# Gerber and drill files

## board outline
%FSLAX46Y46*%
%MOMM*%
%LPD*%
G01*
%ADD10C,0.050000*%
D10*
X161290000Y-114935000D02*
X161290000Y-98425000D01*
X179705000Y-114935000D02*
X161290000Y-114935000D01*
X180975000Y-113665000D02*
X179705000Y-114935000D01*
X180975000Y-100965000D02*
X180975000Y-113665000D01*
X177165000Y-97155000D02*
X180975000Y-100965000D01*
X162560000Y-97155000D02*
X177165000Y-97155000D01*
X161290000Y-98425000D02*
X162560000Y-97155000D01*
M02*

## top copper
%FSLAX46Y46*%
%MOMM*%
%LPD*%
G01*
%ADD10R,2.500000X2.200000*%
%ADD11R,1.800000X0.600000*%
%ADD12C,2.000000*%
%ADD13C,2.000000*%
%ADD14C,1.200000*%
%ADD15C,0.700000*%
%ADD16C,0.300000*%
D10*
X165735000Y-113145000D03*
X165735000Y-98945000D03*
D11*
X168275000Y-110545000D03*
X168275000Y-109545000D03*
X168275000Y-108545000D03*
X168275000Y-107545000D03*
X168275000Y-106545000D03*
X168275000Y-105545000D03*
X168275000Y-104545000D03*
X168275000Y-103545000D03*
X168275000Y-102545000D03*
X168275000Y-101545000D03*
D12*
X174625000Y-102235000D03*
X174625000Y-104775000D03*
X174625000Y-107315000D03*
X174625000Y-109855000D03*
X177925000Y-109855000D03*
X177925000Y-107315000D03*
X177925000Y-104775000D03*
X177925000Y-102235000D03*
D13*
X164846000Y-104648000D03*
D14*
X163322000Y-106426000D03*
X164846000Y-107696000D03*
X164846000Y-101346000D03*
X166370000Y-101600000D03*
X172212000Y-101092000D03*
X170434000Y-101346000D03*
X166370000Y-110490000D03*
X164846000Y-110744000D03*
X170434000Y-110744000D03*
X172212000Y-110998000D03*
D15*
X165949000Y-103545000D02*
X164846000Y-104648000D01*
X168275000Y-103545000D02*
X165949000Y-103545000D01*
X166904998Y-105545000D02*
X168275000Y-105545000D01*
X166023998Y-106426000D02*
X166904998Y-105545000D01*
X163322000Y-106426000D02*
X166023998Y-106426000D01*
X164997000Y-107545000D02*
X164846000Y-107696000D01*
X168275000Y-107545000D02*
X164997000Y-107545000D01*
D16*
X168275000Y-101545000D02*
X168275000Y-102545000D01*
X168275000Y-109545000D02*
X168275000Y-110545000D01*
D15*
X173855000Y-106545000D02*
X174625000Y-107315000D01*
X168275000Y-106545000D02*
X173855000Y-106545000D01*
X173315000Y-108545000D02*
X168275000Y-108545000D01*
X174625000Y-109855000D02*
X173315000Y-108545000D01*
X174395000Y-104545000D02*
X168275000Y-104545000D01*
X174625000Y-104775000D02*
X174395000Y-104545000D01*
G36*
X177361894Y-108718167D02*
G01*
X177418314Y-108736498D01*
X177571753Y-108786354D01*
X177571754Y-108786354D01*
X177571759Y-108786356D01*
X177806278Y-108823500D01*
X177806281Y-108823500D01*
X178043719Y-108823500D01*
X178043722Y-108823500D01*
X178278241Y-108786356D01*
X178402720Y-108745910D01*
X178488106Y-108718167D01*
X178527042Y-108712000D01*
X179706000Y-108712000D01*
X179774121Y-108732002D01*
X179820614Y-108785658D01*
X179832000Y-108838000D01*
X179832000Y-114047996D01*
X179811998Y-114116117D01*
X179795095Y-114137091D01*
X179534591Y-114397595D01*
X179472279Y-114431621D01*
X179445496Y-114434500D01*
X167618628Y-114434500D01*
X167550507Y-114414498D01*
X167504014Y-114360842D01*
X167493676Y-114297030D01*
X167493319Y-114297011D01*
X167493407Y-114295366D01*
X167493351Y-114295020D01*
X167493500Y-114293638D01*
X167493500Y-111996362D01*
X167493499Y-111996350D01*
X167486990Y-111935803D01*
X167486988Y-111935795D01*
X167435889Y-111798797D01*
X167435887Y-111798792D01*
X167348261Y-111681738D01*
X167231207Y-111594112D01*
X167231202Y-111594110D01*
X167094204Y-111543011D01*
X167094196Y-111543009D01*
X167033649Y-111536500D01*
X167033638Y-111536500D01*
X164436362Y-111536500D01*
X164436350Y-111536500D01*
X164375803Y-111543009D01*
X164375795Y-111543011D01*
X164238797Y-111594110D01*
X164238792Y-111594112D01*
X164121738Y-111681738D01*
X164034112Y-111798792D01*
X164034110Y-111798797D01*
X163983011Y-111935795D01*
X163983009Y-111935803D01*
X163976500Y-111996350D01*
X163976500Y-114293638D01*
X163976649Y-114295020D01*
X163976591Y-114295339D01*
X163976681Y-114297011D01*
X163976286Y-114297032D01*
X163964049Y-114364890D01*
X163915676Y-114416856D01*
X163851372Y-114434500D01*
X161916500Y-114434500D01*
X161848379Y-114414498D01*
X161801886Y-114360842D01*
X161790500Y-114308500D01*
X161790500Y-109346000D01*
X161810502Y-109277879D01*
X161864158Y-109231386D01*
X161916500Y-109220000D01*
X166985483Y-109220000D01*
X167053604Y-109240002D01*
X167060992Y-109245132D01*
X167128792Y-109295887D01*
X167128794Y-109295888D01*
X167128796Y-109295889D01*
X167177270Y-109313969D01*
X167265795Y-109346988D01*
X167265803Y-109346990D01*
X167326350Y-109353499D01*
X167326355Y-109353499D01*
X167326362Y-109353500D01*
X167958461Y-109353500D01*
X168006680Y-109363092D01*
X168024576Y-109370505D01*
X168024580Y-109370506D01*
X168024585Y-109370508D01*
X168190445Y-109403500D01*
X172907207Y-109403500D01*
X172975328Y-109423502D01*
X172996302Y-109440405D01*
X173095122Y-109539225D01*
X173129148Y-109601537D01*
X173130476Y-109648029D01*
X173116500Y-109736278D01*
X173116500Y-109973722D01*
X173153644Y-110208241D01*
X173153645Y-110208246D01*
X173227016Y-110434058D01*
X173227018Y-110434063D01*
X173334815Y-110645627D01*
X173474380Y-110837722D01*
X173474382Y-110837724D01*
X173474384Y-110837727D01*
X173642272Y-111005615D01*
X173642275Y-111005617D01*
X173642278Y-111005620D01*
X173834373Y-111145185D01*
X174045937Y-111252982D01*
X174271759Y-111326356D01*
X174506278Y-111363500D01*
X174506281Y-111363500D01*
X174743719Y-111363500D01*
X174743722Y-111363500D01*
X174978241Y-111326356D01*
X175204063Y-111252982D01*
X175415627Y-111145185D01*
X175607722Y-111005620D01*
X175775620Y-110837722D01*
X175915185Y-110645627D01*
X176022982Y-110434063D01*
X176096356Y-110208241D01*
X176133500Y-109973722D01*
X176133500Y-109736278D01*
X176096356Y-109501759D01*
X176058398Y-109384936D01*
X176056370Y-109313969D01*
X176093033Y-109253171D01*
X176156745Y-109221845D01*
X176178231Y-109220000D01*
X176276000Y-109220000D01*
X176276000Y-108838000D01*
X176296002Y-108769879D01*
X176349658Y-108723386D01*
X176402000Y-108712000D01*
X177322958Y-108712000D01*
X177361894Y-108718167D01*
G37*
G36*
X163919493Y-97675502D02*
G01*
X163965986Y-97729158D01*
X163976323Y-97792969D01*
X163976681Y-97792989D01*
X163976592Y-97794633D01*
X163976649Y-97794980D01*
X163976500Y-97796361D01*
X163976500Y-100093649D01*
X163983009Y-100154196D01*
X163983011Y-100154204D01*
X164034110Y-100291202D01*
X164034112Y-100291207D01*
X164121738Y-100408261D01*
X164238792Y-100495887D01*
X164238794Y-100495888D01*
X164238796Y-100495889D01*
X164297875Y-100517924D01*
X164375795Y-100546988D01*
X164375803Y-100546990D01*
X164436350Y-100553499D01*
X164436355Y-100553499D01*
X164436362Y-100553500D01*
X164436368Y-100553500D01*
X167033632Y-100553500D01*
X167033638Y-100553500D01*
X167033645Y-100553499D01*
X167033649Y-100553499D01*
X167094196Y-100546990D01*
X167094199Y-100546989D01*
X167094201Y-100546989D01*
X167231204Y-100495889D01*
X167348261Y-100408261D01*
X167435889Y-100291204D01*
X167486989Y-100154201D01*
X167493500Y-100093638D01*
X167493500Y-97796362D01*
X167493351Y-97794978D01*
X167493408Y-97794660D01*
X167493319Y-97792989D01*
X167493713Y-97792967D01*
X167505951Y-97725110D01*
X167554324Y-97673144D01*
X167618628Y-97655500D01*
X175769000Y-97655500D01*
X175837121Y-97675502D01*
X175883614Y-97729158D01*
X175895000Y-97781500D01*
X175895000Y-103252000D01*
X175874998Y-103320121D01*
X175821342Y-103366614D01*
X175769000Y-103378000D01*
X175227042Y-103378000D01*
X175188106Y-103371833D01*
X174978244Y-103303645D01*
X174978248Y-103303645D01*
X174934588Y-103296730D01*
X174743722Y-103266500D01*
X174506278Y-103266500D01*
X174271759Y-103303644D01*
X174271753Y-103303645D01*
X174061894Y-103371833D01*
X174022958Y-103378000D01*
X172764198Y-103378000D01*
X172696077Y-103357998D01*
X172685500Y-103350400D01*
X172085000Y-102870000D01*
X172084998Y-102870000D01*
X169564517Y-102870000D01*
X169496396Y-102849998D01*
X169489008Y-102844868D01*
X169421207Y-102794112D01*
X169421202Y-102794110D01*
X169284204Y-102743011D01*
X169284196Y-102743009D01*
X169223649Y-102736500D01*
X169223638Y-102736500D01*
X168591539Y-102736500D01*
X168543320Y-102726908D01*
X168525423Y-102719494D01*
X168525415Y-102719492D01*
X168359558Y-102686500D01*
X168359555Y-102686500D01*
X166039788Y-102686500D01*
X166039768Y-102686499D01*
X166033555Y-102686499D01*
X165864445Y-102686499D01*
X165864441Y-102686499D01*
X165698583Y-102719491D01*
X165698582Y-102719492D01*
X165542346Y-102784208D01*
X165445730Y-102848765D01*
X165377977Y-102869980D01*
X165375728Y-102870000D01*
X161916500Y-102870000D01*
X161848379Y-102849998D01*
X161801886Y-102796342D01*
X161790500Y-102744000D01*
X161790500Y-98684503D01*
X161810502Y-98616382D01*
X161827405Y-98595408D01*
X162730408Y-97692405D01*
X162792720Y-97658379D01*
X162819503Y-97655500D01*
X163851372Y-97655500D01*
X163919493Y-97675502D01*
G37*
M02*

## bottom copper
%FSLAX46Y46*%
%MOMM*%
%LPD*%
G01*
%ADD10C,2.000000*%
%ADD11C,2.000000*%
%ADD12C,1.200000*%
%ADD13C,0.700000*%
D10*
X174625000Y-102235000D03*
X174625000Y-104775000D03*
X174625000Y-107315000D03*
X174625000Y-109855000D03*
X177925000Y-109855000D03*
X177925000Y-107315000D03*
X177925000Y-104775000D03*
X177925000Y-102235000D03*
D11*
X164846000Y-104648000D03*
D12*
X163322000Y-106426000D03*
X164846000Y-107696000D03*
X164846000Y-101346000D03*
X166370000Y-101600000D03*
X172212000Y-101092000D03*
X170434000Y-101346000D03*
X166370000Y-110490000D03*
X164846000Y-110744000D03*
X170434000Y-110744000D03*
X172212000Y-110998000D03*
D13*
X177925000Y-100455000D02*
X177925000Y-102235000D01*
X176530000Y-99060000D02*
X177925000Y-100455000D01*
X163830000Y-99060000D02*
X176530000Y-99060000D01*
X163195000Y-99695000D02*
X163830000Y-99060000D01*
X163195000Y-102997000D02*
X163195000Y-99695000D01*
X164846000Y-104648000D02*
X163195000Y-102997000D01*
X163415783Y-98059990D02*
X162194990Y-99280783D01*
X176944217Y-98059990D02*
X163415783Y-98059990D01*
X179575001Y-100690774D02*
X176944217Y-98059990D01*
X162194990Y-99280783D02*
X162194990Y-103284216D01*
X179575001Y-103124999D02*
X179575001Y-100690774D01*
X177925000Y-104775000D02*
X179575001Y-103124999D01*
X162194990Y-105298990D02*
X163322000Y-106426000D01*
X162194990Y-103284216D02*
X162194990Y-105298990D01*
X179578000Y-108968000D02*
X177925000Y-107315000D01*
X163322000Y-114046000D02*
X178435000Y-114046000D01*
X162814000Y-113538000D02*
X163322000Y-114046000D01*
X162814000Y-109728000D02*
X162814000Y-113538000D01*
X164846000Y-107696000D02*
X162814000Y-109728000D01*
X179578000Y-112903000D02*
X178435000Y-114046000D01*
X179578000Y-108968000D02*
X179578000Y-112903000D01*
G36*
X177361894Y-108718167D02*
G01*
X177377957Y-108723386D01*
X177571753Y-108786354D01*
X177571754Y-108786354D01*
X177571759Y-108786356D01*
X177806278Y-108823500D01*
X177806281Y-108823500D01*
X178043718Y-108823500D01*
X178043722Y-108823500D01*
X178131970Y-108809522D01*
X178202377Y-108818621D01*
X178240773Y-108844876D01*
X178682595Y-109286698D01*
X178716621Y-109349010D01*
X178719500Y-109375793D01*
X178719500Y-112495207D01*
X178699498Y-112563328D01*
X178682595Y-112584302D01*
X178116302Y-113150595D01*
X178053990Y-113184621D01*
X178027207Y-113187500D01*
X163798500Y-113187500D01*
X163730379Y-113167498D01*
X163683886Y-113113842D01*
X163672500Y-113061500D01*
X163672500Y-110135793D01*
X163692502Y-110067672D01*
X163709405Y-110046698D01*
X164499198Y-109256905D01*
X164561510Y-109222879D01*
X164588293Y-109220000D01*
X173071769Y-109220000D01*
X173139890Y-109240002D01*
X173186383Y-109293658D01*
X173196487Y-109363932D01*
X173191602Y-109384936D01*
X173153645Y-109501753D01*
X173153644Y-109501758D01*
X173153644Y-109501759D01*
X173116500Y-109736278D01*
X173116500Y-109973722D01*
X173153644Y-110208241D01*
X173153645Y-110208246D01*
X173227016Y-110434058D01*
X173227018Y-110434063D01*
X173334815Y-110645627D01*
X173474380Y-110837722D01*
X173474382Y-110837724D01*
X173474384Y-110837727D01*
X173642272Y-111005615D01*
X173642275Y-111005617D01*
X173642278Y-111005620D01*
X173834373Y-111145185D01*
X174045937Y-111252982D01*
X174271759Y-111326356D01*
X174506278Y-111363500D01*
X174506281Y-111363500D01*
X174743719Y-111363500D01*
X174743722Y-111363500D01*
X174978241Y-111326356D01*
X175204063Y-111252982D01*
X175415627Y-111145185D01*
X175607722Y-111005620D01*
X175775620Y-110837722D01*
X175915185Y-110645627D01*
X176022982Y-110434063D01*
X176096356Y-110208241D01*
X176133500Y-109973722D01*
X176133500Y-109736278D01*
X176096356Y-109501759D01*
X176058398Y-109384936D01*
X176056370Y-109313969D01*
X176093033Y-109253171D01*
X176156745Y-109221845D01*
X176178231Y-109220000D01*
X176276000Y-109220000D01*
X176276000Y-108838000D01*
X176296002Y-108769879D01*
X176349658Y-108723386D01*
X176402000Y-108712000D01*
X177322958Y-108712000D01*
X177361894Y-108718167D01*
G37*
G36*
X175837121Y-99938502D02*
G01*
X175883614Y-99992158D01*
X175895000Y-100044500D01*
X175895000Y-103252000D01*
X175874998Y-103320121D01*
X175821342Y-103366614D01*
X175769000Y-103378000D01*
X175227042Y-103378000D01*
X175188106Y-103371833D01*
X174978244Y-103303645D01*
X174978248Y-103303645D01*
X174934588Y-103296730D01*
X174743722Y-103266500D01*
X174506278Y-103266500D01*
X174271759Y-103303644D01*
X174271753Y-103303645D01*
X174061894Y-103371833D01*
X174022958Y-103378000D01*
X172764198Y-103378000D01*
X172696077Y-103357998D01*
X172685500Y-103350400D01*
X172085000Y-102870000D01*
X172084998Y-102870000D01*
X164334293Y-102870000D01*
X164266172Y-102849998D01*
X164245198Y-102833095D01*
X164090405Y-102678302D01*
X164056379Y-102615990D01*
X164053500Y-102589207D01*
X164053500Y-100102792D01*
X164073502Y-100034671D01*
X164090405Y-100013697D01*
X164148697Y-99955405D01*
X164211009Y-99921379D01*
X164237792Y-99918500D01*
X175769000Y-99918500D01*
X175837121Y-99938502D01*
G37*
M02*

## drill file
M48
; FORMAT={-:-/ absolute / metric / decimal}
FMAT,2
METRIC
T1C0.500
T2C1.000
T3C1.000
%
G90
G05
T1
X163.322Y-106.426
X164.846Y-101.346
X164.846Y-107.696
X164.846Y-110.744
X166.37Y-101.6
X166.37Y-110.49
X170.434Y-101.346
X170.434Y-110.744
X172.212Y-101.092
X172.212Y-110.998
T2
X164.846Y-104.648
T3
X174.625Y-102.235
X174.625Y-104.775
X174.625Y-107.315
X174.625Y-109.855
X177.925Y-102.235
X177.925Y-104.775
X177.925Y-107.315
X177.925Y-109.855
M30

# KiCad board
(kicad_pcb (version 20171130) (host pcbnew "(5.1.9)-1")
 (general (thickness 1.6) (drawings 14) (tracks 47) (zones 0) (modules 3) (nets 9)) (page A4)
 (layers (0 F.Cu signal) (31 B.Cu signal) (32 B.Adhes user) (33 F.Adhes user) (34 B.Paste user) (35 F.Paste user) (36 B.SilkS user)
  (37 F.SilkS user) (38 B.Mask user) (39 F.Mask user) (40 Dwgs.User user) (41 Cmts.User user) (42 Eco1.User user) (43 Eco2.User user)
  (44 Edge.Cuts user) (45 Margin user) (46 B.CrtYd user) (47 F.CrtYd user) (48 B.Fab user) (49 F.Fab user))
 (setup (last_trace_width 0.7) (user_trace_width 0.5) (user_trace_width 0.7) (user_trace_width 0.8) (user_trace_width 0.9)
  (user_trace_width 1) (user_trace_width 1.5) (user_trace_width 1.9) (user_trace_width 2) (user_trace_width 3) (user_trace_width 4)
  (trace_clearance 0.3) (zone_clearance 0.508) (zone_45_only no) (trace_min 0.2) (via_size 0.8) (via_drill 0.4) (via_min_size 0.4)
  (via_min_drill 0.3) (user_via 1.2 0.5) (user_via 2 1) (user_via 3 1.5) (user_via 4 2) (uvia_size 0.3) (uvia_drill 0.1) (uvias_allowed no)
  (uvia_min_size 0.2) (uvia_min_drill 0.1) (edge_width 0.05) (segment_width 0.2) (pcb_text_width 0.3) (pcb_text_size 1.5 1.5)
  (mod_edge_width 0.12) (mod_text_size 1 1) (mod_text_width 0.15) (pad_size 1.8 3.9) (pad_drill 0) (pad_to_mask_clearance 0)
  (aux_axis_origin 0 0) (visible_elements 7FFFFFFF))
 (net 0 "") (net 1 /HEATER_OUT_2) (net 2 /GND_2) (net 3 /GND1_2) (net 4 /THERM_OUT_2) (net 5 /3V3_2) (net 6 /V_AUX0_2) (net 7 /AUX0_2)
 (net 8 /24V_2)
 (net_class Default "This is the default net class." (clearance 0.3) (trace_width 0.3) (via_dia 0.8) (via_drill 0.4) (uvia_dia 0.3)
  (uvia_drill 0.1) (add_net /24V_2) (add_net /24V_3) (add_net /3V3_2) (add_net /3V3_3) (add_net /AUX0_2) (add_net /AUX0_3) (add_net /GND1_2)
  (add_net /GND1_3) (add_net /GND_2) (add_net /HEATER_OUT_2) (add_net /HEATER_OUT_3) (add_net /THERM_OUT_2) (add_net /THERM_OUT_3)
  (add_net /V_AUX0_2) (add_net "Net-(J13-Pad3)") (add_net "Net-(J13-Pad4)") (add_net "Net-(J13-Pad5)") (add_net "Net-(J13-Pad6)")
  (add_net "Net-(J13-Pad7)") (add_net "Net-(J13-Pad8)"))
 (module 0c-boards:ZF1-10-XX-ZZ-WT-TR (layer F.Cu) (at 168.275 106.045 270)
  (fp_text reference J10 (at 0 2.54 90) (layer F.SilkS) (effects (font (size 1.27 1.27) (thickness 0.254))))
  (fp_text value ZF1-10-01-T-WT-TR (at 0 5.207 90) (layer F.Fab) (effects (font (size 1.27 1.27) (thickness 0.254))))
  (pad 12 smd rect (at 7.1 2.54 270) (size 2.2 2.5) (layers F.Cu F.Paste F.Mask))
  (pad 11 smd rect (at -7.1 2.54 270) (size 2.2 2.5) (layers F.Cu F.Paste F.Mask))
  (pad 10 smd rect (at 4.5 0 270) (size 0.6 1.8) (layers F.Cu F.Paste F.Mask) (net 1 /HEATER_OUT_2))
  (pad 9 smd rect (at 3.5 0 270) (size 0.6 1.8) (layers F.Cu F.Paste F.Mask) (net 1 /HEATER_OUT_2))
  (pad 8 smd rect (at 2.5 0 270) (size 0.6 1.8) (layers F.Cu F.Paste F.Mask) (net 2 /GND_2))
  (pad 7 smd rect (at 1.5 0 270) (size 0.6 1.8) (layers F.Cu F.Paste F.Mask) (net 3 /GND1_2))
  (pad 6 smd rect (at 0.5 0 270) (size 0.6 1.8) (layers F.Cu F.Paste F.Mask) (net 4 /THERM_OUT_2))
  (pad 5 smd rect (at -0.5 0 270) (size 0.6 1.8) (layers F.Cu F.Paste F.Mask) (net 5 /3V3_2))
  (pad 4 smd rect (at -1.5 0 270) (size 0.6 1.8) (layers F.Cu F.Paste F.Mask) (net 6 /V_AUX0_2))
  (pad 3 smd rect (at -2.5 0 270) (size 0.6 1.8) (layers F.Cu F.Paste F.Mask) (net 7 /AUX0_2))
  (pad 2 smd rect (at -3.5 0 270) (size 0.6 1.8) (layers F.Cu F.Paste F.Mask) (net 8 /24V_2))
  (pad 1 smd rect (at -4.5 0 270) (size 0.6 1.8) (layers F.Cu F.Paste F.Mask) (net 8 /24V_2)))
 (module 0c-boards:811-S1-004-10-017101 (layer B.Cu) (at 174.625 106.045 270)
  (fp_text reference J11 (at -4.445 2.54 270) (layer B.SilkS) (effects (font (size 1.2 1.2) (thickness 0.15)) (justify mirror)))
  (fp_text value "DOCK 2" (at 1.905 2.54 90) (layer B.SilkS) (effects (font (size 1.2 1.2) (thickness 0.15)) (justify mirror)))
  (pad 1 thru_hole circle (at -3.81 0 270) (size 2 2) (drill 1) (layers *.Cu *.Mask) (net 8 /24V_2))
  (pad 2 thru_hole circle (at -1.27 0 270) (size 2 2) (drill 1) (layers *.Cu *.Mask) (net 6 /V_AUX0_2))
  (pad 3 thru_hole circle (at 1.27 0 270) (size 2 2) (drill 1) (layers *.Cu *.Mask) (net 4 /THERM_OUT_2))
  (pad 4 thru_hole circle (at 3.81 0 270) (size 2 2) (drill 1) (layers *.Cu *.Mask) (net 2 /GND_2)))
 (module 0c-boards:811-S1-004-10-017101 (layer B.Cu) (at 177.925 106.045 90)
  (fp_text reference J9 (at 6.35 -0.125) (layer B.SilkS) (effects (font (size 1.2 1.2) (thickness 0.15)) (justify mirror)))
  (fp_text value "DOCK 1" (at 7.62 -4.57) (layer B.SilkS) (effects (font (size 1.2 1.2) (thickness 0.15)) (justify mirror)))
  (pad 1 thru_hole circle (at -3.81 0 90) (size 2 2) (drill 1) (layers *.Cu *.Mask) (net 1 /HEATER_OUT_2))
  (pad 2 thru_hole circle (at -1.27 0 90) (size 2 2) (drill 1) (layers *.Cu *.Mask) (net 3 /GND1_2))
  (pad 3 thru_hole circle (at 1.27 0 90) (size 2 2) (drill 1) (layers *.Cu *.Mask) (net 5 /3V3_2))
  (pad 4 thru_hole circle (at 3.81 0 90) (size 2 2) (drill 1) (layers *.Cu *.Mask) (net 7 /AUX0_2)))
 (gr_line (start 161.29 114.935) (end 161.29 98.425) (layer Edge.Cuts) (width 0.05))
 (gr_line (start 179.705 114.935) (end 161.29 114.935) (layer Edge.Cuts) (width 0.05))
 (gr_line (start 180.975 113.665) (end 179.705 114.935) (layer Edge.Cuts) (width 0.05))
 (gr_line (start 180.975 100.965) (end 180.975 113.665) (layer Edge.Cuts) (width 0.05))
 (gr_line (start 177.165 97.155) (end 180.975 100.965) (layer Edge.Cuts) (width 0.05))
 (gr_line (start 162.56 97.155) (end 177.165 97.155) (layer Edge.Cuts) (width 0.05))
 (gr_line (start 161.29 98.425) (end 162.56 97.155) (layer Edge.Cuts) (width 0.05))
 (via (at 164.846 104.648) (size 2) (drill 1) (layers F.Cu B.Cu) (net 7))
 (segment (start 165.949 103.545) (end 164.846 104.648) (width 0.7) (layer F.Cu) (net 7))
 (segment (start 168.275 103.545) (end 165.949 103.545) (width 0.7) (layer F.Cu) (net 7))
 (segment (start 177.925 100.455) (end 177.925 102.235) (width 0.7) (layer B.Cu) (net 7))
 (segment (start 176.53 99.06) (end 177.925 100.455) (width 0.7) (layer B.Cu) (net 7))
 (segment (start 163.83 99.06) (end 176.53 99.06) (width 0.7) (layer B.Cu) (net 7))
 (segment (start 163.195 99.695) (end 163.83 99.06) (width 0.7) (layer B.Cu) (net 7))
 (segment (start 163.195 102.997) (end 163.195 99.695) (width 0.7) (layer B.Cu) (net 7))
 (segment (start 164.846 104.648) (end 163.195 102.997) (width 0.7) (layer B.Cu) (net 7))
 (segment (start 163.415783 98.05999) (end 162.19499 99.280783) (width 0.7) (layer B.Cu) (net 5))
 (segment (start 176.944217 98.05999) (end 163.415783 98.05999) (width 0.7) (layer B.Cu) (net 5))
 (segment (start 179.575001 100.690774) (end 176.944217 98.05999) (width 0.7) (layer B.Cu) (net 5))
 (segment (start 162.19499 99.280783) (end 162.19499 103.284216) (width 0.7) (layer B.Cu) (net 5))
 (segment (start 179.575001 103.124999) (end 179.575001 100.690774) (width 0.7) (layer B.Cu) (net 5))
 (segment (start 177.925 104.775) (end 179.575001 103.124999) (width 0.7) (layer B.Cu) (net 5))
 (via (at 163.322 106.426) (size 1.2) (drill 0.5) (layers F.Cu B.Cu) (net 5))
 (segment (start 162.19499 105.29899) (end 163.322 106.426) (width 0.7) (layer B.Cu) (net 5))
 (segment (start 162.19499 103.284216) (end 162.19499 105.29899) (width 0.7) (layer B.Cu) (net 5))
 (segment (start 166.904998 105.545) (end 168.275 105.545) (width 0.7) (layer F.Cu) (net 5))
 (segment (start 166.023998 106.426) (end 166.904998 105.545) (width 0.7) (layer F.Cu) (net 5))
 (segment (start 163.322 106.426) (end 166.023998 106.426) (width 0.7) (layer F.Cu) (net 5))
 (via (at 164.846 107.696) (size 1.2) (drill 0.5) (layers F.Cu B.Cu) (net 3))
 (segment (start 164.997 107.545) (end 164.846 107.696) (width 0.7) (layer F.Cu) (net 3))
 (segment (start 168.275 107.545) (end 164.997 107.545) (width 0.7) (layer F.Cu) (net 3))
 (segment (start 179.578 108.968) (end 177.925 107.315) (width 0.7) (layer B.Cu) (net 3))
 (segment (start 163.322 114.046) (end 178.435 114.046) (width 0.7) (layer B.Cu) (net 3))
 (segment (start 162.814 113.538) (end 163.322 114.046) (width 0.7) (layer B.Cu) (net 3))
 (segment (start 162.814 109.728) (end 162.814 113.538) (width 0.7) (layer B.Cu) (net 3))
 (segment (start 164.846 107.696) (end 162.814 109.728) (width 0.7) (layer B.Cu) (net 3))
 (segment (start 179.578 112.903) (end 178.435 114.046) (width 0.7) (layer B.Cu) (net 3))
 (segment (start 179.578 108.968) (end 179.578 112.903) (width 0.7) (layer B.Cu) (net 3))
 (segment (start 168.275 101.545) (end 168.275 102.545) (width 0.3) (layer F.Cu) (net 8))
 (via (at 164.846 101.346) (size 1.2) (drill 0.5) (layers F.Cu B.Cu) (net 8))
 (via (at 166.37 101.6) (size 1.2) (drill 0.5) (layers F.Cu B.Cu) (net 8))
 (via (at 172.212 101.092) (size 1.2) (drill 0.5) (layers F.Cu B.Cu) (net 8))
 (via (at 170.434 101.346) (size 1.2) (drill 0.5) (layers F.Cu B.Cu) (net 8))
 (via (at 166.37 110.49) (size 1.2) (drill 0.5) (layers F.Cu B.Cu) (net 1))
 (segment (start 168.275 109.545) (end 168.275 110.545) (width 0.3) (layer F.Cu) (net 1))
 (via (at 164.846 110.744) (size 1.2) (drill 0.5) (layers F.Cu B.Cu) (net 1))
 (via (at 170.434 110.744) (size 1.2) (drill 0.5) (layers F.Cu B.Cu) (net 1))
 (via (at 172.212 110.998) (size 1.2) (drill 0.5) (layers F.Cu B.Cu) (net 1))
 (segment (start 173.855 106.545) (end 174.625 107.315) (width 0.7) (layer F.Cu) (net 4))
 (segment (start 168.275 106.545) (end 173.855 106.545) (width 0.7) (layer F.Cu) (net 4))
 (segment (start 173.315 108.545) (end 168.275 108.545) (width 0.7) (layer F.Cu) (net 2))
 (segment (start 174.625 109.855) (end 173.315 108.545) (width 0.7) (layer F.Cu) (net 2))
 (segment (start 174.395 104.545) (end 168.275 104.545) (width 0.7) (layer F.Cu) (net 6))
 (segment (start 174.625 104.775) (end 174.395 104.545) (width 0.7) (layer F.Cu) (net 6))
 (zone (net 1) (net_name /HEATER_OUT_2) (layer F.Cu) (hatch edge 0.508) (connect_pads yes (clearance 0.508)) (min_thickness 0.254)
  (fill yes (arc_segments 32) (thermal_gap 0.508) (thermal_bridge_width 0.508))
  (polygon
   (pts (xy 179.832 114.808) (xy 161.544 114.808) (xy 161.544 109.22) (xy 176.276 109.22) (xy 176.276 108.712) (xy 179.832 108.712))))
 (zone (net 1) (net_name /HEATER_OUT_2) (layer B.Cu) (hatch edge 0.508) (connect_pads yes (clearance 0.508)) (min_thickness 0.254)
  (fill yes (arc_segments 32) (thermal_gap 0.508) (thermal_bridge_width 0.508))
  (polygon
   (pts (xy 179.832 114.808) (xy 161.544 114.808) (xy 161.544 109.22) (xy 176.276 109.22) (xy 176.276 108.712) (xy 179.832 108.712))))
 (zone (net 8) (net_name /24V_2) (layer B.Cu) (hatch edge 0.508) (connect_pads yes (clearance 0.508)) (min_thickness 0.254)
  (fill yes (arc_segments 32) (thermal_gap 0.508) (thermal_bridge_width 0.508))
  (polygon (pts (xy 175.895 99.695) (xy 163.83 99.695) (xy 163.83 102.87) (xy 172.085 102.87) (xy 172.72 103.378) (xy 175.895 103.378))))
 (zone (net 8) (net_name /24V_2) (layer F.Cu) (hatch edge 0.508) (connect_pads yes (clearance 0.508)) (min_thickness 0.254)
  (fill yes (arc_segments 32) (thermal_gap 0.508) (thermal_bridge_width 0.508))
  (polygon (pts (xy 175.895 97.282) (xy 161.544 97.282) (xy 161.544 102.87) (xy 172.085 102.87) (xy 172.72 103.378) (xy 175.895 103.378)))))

